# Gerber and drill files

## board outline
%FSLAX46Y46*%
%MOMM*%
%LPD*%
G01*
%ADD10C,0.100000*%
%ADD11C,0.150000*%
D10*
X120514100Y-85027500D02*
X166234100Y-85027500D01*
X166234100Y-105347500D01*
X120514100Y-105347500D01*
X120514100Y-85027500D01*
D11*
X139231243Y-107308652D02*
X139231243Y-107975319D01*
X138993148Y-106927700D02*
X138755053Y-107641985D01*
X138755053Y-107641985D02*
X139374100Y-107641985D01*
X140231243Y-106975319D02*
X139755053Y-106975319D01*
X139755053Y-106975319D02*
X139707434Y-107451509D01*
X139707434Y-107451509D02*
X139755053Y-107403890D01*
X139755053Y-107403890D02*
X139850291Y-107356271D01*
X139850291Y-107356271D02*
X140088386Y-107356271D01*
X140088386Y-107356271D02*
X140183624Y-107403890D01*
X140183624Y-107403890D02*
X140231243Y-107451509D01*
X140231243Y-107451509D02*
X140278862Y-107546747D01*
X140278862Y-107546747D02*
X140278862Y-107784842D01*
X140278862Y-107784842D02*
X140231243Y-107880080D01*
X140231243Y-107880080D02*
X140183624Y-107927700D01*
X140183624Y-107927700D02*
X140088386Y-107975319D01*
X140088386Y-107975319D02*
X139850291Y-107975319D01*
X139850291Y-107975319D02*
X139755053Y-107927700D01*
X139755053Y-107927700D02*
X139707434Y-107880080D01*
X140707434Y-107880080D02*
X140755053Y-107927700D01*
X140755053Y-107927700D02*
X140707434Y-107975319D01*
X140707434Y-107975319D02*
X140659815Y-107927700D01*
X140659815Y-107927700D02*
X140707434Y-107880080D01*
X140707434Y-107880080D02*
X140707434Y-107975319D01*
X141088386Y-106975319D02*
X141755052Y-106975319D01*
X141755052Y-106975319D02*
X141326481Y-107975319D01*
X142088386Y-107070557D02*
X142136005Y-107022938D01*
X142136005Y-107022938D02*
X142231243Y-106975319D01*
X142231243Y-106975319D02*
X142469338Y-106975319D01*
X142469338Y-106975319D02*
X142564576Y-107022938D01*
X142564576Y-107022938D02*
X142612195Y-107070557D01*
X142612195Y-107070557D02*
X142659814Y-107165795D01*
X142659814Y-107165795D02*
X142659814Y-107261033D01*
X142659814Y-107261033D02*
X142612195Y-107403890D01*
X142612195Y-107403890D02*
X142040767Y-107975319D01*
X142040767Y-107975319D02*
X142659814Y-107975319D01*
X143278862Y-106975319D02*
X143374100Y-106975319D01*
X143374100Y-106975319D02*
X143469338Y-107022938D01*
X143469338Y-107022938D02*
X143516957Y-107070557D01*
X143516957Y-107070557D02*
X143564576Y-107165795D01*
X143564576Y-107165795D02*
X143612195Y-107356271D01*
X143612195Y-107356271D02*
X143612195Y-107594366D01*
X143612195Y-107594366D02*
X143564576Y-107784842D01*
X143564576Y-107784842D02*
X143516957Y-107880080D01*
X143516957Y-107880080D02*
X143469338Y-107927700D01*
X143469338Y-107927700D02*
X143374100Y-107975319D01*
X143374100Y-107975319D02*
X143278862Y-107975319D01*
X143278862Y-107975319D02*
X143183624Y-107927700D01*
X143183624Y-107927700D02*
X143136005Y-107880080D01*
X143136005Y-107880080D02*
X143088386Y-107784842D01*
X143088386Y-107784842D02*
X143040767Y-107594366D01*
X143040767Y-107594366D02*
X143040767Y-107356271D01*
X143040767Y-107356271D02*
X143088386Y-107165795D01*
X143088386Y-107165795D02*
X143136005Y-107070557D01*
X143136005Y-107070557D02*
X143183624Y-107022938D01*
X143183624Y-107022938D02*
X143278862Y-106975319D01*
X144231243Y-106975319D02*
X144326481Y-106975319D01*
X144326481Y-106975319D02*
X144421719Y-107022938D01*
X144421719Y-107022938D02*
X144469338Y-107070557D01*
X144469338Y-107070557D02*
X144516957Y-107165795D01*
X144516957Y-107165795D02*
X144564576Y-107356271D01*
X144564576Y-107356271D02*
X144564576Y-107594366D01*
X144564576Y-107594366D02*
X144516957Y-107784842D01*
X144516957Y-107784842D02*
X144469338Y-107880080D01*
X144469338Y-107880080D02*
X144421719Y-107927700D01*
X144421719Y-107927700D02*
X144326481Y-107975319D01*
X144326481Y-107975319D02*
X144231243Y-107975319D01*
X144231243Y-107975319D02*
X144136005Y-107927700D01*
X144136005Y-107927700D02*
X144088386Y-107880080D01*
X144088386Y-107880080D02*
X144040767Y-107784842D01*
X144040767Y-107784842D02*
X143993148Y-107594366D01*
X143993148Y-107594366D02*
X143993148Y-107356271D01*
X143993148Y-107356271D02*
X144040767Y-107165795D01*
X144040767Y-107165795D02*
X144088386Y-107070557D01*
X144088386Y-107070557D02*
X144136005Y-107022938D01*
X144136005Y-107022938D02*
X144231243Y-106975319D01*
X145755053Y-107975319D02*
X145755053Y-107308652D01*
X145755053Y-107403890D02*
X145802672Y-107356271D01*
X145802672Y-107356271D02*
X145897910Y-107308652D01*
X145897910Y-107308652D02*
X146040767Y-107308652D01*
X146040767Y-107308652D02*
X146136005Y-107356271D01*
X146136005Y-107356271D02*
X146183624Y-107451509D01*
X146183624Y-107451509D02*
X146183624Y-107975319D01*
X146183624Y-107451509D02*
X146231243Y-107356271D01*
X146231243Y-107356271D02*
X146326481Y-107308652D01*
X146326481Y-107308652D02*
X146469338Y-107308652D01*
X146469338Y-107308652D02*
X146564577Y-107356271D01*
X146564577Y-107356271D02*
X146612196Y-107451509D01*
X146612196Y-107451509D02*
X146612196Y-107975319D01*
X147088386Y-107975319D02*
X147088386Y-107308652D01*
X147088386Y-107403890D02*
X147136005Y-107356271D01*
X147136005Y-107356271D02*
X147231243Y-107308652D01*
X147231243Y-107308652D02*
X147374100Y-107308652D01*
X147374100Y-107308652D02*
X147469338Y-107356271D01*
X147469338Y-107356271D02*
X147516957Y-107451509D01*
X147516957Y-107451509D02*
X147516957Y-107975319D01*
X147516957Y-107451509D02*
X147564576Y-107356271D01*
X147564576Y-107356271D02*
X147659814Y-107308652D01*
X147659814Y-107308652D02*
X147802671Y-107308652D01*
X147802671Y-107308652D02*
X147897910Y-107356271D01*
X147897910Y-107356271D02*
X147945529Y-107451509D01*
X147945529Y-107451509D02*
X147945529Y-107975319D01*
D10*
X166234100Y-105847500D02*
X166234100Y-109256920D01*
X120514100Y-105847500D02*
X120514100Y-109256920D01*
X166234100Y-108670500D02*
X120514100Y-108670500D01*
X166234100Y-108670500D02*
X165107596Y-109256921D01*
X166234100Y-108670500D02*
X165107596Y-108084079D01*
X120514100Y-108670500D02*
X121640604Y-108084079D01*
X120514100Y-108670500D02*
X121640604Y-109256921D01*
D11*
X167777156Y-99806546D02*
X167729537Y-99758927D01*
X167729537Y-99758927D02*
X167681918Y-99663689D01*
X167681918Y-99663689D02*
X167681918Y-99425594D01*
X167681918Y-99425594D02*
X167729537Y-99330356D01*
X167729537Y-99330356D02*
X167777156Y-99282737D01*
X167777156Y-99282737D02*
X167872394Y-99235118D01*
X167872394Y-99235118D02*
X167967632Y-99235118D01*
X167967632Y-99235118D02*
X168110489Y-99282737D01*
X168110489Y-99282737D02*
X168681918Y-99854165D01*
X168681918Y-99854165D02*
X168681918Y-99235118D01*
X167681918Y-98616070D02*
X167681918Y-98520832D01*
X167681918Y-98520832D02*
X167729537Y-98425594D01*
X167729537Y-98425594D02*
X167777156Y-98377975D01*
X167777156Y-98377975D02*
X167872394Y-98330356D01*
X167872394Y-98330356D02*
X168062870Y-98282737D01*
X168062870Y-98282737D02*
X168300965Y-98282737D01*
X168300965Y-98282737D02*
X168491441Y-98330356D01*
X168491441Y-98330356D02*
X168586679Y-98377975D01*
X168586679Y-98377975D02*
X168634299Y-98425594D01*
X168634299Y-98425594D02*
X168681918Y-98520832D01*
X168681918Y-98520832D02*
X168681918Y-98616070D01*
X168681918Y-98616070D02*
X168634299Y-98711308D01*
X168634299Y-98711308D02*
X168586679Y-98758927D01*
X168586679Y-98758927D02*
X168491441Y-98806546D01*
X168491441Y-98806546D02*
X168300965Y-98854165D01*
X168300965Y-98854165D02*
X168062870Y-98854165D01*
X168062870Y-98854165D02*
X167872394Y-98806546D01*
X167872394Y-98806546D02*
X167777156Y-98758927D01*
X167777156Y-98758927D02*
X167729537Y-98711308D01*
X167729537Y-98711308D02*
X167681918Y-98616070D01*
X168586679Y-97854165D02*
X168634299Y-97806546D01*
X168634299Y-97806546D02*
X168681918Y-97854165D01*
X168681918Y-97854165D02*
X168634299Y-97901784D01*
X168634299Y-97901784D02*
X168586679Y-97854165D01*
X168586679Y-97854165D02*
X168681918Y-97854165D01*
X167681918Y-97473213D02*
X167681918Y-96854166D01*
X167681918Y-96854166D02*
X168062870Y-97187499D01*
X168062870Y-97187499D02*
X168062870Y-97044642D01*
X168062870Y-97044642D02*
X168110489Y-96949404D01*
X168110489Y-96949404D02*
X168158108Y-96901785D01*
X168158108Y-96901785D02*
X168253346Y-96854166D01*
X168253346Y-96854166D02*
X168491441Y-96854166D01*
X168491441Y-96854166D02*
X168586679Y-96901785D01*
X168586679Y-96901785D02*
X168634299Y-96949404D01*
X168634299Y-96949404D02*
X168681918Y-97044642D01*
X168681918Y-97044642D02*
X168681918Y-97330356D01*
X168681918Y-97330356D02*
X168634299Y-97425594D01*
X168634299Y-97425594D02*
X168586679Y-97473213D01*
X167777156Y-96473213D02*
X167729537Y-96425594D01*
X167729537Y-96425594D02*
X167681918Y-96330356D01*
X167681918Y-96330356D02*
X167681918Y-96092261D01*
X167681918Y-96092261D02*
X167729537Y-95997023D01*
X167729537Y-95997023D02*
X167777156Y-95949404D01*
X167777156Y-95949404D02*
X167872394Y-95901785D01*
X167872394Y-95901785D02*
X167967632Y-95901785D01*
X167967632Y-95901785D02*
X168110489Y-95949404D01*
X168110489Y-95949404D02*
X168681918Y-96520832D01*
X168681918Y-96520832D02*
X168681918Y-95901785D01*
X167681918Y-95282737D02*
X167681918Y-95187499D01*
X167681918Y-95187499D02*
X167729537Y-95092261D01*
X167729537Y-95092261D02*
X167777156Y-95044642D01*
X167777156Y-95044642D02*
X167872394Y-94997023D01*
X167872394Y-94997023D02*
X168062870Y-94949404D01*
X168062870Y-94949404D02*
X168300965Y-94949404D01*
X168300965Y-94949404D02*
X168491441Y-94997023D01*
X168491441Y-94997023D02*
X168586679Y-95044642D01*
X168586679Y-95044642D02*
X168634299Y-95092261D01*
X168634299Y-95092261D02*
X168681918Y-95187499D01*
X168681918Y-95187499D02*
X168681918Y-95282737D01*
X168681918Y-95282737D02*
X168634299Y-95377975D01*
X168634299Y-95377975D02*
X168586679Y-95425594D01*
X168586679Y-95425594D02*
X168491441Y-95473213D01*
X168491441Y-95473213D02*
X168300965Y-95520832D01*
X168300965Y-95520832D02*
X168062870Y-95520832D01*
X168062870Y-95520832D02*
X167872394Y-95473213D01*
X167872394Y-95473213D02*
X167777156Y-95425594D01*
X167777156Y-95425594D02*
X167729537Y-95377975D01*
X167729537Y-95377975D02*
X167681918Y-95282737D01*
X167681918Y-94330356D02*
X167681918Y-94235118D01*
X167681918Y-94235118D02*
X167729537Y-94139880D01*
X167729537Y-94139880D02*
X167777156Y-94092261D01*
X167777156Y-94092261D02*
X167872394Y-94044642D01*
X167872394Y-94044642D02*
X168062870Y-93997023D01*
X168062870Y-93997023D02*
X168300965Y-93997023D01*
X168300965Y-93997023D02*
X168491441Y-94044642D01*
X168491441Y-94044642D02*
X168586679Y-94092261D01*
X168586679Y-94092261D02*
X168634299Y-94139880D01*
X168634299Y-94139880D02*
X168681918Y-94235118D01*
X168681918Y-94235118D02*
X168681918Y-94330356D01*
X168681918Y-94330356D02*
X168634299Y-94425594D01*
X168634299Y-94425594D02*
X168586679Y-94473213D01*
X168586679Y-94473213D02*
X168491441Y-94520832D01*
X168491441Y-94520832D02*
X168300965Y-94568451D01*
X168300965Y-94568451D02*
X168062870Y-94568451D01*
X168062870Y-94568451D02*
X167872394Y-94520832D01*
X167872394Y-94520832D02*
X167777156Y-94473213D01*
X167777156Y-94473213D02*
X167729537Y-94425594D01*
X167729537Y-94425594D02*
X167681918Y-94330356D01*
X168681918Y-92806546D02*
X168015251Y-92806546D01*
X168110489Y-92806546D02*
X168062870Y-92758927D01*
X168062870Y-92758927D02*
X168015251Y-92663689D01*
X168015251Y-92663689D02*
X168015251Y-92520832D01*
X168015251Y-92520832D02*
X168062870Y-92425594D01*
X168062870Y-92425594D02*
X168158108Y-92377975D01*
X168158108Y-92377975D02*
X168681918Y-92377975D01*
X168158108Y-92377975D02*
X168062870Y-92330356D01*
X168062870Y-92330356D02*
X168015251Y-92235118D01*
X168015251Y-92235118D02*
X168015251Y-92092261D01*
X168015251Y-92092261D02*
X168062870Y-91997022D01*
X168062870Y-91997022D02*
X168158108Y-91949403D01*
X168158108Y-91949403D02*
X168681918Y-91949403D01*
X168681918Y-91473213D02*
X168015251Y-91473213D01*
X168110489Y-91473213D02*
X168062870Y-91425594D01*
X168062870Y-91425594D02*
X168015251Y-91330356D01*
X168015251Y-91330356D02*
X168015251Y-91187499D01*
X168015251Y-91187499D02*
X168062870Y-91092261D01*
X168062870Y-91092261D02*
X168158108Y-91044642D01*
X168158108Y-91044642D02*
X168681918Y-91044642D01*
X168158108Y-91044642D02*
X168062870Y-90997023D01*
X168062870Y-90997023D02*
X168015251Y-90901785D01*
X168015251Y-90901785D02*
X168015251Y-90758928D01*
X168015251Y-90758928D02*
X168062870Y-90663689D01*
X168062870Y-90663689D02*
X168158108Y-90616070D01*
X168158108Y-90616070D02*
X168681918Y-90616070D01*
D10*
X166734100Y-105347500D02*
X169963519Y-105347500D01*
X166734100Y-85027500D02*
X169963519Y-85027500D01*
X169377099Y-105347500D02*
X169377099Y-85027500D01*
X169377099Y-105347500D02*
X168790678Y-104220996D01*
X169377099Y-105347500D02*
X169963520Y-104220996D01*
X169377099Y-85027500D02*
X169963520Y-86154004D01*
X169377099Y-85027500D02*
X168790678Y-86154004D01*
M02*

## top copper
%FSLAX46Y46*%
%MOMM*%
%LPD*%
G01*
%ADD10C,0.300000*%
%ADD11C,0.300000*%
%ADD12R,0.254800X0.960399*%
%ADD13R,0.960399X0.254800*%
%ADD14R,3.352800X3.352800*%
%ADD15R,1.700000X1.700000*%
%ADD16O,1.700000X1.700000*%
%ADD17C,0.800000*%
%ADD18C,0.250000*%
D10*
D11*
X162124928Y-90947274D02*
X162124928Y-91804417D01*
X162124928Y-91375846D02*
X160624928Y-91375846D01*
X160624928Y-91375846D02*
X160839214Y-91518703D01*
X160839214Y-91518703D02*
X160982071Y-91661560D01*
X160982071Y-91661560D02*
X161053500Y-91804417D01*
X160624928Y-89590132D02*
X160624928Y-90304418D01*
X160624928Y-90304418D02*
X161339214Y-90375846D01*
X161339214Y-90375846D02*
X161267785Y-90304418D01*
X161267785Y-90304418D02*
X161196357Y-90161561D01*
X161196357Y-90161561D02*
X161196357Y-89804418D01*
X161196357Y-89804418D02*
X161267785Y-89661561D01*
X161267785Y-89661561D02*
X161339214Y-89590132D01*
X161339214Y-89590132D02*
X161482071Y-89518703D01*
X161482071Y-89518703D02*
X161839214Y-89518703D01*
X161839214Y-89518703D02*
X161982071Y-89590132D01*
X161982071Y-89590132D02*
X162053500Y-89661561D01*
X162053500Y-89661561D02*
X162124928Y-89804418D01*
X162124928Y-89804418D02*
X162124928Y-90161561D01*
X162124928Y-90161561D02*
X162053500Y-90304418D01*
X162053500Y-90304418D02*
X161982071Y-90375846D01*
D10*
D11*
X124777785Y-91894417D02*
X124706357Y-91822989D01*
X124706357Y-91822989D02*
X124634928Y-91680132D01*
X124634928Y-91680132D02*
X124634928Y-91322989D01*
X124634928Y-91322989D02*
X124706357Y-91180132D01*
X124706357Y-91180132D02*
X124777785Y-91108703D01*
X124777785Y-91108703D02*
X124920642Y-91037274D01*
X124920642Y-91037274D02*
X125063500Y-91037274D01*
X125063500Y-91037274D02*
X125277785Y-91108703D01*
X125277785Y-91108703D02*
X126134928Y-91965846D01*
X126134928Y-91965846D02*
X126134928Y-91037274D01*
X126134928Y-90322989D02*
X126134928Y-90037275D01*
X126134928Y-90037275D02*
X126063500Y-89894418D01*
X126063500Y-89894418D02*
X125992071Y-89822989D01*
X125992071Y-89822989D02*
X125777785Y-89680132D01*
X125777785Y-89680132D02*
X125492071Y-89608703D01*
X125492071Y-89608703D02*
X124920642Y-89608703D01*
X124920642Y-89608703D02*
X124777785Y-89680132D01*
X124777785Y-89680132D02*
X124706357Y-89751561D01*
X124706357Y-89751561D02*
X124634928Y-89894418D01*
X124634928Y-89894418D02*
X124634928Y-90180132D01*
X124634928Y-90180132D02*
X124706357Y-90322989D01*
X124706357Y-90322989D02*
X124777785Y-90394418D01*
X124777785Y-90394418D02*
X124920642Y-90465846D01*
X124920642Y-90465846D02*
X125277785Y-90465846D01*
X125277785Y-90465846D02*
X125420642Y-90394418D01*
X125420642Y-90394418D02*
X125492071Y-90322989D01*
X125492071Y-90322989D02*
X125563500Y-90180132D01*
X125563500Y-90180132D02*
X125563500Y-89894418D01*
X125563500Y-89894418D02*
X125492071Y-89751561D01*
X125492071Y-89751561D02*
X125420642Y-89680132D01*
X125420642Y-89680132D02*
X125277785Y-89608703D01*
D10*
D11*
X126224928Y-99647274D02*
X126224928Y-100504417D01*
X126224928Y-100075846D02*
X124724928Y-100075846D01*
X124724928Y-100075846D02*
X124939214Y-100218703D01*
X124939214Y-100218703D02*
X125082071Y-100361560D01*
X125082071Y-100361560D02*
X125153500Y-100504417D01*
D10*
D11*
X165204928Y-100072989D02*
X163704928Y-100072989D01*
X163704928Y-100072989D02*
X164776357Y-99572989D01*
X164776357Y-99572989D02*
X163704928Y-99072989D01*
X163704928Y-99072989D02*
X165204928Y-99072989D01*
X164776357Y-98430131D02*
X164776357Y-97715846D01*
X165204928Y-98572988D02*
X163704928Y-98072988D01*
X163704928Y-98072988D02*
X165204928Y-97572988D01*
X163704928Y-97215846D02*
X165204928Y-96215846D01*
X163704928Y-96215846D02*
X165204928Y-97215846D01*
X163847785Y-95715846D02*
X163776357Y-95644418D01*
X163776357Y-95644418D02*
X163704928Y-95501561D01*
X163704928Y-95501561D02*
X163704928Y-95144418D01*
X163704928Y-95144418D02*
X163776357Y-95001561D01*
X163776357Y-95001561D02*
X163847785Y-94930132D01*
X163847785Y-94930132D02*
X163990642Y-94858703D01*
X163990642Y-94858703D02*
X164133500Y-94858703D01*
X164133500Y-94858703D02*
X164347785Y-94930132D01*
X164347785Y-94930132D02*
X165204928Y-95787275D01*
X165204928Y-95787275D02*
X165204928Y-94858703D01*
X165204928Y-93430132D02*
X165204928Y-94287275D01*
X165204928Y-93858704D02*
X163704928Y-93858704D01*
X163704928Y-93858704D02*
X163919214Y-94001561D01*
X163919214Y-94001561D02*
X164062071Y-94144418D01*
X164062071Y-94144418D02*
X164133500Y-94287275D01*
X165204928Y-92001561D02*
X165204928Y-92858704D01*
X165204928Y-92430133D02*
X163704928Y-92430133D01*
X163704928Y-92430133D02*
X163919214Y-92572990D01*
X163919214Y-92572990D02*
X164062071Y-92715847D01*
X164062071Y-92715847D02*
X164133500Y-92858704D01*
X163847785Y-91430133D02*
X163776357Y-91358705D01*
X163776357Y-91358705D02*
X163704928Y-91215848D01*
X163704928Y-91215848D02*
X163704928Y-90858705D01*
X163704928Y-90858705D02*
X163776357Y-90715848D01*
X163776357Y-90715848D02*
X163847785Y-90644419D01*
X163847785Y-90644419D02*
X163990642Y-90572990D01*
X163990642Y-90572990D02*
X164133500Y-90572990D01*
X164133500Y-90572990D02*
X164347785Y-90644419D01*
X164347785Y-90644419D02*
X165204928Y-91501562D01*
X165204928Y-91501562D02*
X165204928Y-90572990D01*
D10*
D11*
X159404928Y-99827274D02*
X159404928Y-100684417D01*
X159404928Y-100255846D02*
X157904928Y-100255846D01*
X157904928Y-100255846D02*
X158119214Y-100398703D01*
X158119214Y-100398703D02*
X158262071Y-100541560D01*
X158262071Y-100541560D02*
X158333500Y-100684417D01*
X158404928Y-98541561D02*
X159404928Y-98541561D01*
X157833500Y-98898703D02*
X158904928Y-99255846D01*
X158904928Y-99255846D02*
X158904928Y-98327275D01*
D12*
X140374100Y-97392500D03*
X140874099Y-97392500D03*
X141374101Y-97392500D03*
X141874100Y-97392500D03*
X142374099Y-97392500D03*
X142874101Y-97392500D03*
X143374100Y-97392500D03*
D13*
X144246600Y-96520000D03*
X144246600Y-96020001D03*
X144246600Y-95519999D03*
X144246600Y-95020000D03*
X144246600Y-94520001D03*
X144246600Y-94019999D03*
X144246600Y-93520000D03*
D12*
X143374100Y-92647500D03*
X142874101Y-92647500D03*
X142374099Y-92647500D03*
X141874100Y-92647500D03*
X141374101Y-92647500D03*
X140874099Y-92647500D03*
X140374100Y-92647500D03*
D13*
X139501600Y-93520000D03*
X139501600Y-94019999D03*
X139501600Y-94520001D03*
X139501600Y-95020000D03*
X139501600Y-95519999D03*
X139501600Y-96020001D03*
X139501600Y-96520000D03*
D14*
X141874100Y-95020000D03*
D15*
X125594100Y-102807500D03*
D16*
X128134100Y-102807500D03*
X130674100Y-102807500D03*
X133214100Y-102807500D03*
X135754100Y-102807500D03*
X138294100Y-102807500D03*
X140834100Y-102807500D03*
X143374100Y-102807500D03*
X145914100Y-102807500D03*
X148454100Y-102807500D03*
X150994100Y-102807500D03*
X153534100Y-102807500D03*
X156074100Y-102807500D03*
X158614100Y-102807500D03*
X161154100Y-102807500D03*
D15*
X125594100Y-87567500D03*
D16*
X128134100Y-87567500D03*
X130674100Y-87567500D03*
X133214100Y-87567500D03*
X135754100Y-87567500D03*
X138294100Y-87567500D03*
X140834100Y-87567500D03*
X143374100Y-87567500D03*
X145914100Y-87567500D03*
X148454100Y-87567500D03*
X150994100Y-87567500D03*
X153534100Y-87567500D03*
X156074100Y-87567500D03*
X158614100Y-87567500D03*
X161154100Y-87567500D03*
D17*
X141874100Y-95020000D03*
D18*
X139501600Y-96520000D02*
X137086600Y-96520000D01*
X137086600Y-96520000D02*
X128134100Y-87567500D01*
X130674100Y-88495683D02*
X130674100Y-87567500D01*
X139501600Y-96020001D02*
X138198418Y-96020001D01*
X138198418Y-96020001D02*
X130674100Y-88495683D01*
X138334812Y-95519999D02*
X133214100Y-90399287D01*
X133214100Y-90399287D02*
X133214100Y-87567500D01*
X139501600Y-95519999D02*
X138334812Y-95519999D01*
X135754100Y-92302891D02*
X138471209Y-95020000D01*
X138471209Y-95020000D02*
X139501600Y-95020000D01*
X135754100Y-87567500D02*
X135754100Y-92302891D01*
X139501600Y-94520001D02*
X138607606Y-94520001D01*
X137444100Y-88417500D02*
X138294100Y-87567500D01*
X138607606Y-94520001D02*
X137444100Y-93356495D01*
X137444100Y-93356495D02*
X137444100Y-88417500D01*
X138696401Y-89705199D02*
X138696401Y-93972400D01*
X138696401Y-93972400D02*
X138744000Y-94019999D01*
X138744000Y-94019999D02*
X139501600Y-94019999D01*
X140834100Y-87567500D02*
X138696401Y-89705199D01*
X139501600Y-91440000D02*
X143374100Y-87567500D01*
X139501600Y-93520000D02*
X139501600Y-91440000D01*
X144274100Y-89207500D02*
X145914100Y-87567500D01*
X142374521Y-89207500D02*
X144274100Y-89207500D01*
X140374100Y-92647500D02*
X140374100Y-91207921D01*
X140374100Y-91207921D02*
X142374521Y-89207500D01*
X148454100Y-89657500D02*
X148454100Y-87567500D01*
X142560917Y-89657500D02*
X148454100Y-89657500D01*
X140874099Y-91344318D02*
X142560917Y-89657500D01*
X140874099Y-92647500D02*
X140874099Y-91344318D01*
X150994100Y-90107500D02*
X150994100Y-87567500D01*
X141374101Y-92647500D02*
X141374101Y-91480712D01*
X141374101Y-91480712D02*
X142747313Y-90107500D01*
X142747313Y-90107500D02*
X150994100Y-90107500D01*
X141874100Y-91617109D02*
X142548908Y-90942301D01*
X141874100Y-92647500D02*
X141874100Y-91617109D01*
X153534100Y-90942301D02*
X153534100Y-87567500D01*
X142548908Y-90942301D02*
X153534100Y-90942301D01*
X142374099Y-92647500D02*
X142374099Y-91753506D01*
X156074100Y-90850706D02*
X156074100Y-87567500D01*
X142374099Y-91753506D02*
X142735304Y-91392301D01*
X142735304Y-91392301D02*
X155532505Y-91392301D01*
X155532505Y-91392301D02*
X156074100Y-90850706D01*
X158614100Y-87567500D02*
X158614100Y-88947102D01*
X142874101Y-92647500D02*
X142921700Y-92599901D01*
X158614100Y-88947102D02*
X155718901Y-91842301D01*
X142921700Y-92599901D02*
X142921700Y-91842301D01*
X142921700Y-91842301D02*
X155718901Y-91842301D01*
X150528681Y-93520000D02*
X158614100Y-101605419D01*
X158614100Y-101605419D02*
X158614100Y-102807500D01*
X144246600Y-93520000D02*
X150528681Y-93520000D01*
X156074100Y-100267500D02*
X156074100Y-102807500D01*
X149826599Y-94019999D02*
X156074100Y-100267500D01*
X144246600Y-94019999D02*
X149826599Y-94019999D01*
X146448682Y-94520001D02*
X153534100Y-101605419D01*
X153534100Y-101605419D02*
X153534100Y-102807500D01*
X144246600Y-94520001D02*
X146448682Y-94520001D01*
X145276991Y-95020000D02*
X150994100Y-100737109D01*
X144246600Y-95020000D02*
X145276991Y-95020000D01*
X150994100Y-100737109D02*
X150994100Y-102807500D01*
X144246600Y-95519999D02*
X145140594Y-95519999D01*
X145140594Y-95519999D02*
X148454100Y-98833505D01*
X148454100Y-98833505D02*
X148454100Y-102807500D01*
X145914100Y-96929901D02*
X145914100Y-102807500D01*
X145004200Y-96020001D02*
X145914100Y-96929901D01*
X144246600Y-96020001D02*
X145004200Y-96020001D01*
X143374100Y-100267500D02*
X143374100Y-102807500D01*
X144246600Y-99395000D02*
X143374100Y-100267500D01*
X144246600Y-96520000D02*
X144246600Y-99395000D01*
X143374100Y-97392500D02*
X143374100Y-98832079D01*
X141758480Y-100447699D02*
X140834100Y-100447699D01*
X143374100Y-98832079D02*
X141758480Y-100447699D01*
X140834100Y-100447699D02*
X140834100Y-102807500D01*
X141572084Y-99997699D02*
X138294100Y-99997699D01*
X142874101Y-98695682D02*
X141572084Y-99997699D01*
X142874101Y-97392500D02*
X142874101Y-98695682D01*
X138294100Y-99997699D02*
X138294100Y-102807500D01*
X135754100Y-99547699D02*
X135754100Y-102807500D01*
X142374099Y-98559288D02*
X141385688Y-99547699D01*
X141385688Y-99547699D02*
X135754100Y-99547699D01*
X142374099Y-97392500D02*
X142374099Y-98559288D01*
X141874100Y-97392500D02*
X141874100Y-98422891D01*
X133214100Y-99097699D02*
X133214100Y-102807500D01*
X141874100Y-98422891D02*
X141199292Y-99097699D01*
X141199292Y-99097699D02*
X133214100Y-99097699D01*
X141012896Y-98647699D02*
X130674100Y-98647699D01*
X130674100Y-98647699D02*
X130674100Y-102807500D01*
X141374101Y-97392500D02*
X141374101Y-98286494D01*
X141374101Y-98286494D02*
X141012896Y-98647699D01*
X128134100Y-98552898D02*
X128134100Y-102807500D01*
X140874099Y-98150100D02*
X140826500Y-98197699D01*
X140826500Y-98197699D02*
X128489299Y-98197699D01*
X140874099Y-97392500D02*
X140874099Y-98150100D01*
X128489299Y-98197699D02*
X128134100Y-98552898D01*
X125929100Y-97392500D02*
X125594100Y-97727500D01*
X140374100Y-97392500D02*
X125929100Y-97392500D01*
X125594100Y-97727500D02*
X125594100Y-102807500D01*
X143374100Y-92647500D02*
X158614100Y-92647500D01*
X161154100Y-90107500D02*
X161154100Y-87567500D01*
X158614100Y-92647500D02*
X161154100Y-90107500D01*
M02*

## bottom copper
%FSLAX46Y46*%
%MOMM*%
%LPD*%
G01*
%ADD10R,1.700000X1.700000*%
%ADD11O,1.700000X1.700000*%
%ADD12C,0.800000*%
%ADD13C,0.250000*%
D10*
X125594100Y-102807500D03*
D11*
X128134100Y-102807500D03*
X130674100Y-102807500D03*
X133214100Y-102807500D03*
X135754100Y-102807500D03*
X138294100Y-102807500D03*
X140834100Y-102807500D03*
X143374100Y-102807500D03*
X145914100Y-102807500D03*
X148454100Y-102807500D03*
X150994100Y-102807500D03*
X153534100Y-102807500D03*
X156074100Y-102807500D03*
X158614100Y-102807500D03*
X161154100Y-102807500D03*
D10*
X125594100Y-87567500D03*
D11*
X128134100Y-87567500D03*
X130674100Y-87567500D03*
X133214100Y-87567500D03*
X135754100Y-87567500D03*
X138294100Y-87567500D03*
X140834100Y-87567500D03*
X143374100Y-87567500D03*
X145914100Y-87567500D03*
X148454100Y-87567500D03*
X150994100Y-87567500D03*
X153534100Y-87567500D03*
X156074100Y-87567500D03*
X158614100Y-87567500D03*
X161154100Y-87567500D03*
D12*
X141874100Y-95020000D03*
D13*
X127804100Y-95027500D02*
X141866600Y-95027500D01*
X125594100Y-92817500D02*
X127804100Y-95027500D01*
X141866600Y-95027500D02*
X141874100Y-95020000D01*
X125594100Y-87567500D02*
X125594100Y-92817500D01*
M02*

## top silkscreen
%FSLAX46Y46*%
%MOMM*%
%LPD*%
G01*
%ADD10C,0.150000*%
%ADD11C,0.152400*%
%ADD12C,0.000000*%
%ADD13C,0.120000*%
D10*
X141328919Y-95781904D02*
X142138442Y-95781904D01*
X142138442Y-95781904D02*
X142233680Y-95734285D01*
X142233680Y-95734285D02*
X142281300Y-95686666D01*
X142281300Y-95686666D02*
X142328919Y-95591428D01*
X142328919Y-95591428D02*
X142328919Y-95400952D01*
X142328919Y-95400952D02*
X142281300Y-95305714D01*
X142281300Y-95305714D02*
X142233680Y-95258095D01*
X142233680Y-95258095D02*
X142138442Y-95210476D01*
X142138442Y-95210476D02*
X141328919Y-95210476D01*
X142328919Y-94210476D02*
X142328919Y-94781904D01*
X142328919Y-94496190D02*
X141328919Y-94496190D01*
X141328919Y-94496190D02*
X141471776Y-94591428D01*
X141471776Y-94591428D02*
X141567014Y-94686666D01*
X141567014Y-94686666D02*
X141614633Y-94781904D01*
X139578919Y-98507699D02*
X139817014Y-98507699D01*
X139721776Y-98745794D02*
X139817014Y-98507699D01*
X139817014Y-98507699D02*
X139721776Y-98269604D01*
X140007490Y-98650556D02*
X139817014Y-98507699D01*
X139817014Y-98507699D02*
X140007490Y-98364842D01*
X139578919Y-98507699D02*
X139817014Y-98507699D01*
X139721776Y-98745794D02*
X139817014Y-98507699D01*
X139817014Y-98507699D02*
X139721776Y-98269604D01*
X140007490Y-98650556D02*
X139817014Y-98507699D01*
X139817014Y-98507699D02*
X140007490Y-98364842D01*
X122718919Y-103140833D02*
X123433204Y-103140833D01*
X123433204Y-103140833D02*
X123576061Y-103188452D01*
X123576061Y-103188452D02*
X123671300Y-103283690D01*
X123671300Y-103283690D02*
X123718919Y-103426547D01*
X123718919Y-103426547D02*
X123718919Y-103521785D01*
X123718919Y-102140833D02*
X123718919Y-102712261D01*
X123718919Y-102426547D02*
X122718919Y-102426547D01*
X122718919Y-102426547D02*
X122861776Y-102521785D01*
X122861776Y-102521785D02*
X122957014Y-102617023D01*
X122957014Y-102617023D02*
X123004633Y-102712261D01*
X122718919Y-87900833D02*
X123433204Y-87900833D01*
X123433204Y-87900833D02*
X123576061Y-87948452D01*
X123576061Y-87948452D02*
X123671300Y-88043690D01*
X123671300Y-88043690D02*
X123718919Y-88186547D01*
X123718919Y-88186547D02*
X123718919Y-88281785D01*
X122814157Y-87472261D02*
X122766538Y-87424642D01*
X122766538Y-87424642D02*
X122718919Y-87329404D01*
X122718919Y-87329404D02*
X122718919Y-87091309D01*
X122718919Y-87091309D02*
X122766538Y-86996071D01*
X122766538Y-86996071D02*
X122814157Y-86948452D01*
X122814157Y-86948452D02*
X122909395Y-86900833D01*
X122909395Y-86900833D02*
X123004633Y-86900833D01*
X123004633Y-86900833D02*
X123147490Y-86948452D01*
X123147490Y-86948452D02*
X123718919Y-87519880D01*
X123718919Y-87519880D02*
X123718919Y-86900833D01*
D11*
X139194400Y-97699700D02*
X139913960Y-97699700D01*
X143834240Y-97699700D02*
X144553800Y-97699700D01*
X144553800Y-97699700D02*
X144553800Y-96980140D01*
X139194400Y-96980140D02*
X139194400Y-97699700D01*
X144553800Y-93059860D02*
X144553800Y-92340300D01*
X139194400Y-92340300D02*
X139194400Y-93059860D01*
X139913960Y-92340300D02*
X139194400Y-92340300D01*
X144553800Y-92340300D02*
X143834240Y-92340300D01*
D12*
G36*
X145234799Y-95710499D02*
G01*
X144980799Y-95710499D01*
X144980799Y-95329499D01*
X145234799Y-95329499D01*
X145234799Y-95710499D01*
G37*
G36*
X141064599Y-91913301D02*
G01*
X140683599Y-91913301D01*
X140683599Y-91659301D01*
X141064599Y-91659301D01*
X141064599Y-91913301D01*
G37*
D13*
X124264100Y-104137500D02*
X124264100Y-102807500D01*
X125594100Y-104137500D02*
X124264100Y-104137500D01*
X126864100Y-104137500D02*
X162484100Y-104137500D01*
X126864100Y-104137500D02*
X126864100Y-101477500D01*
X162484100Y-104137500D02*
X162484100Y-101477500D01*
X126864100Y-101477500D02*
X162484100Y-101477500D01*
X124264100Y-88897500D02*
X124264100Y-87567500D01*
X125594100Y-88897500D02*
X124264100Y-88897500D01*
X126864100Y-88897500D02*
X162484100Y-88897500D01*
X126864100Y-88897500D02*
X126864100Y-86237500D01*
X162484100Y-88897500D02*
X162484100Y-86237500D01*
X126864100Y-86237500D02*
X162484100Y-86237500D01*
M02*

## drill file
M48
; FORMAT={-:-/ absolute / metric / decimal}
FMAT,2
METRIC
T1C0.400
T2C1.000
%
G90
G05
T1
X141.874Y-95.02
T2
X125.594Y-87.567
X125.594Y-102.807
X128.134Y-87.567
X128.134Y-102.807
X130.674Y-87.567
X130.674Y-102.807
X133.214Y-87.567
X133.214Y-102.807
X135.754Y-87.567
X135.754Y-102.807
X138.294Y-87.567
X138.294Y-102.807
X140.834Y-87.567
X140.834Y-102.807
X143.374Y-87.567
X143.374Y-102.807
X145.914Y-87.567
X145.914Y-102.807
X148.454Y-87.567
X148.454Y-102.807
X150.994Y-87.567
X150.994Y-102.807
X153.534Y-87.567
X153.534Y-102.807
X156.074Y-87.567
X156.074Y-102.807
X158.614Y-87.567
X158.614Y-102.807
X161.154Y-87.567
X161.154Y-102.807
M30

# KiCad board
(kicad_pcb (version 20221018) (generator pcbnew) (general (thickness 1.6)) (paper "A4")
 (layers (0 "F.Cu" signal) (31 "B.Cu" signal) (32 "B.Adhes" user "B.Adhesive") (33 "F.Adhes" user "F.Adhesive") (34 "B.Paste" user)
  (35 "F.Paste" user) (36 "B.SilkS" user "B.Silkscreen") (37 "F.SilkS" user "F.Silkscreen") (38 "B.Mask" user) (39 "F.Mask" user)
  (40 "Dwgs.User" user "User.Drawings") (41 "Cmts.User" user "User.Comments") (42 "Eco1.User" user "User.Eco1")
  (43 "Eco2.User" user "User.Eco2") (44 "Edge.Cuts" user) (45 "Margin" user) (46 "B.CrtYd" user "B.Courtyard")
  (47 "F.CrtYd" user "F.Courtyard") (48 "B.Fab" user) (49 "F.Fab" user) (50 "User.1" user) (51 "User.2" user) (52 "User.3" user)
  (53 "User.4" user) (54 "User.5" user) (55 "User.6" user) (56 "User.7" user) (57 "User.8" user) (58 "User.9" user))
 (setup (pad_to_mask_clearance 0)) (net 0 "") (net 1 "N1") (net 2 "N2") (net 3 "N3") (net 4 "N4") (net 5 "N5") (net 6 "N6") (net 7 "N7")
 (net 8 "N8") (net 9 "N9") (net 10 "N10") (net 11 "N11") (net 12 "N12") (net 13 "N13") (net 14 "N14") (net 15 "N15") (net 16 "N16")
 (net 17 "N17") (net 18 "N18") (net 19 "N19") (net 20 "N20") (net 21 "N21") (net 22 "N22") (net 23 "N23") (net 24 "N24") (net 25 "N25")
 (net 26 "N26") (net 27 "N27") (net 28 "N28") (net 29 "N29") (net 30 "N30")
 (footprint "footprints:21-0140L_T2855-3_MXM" (layer "F.Cu") (at 141.8741 95.02 90)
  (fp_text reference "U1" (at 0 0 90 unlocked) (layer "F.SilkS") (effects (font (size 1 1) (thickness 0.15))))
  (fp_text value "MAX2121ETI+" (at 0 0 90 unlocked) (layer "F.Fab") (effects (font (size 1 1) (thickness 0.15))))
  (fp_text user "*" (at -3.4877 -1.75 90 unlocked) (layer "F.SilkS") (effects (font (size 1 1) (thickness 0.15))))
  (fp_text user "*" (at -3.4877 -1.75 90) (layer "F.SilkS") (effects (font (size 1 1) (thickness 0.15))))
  (fp_line (start -2.6797 -2.6797) (end -2.6797 -1.96014) (stroke (width 0.1524) (type solid)) (layer "F.SilkS"))
  (fp_line (start -2.6797 1.96014) (end -2.6797 2.6797) (stroke (width 0.1524) (type solid)) (layer "F.SilkS"))
  (fp_line (start -2.6797 2.6797) (end -1.96014 2.6797) (stroke (width 0.1524) (type solid)) (layer "F.SilkS"))
  (fp_line (start -1.96014 -2.6797) (end -2.6797 -2.6797) (stroke (width 0.1524) (type solid)) (layer "F.SilkS"))
  (fp_line (start 1.96014 2.6797) (end 2.6797 2.6797) (stroke (width 0.1524) (type solid)) (layer "F.SilkS"))
  (fp_line (start 2.6797 -2.6797) (end 1.96014 -2.6797) (stroke (width 0.1524) (type solid)) (layer "F.SilkS"))
  (fp_line (start 2.6797 -1.96014) (end 2.6797 -2.6797) (stroke (width 0.1524) (type solid)) (layer "F.SilkS"))
  (fp_line (start 2.6797 2.6797) (end 2.6797 1.96014) (stroke (width 0.1524) (type solid)) (layer "F.SilkS"))
  (fp_poly
   (pts (xy -0.690499 3.106699) (xy -0.690499 3.360699) (xy -0.309499 3.360699) (xy -0.309499 3.106699)) (stroke (width 0) (type solid))
   (fill solid) (layer "F.SilkS"))
  (fp_poly
   (pts (xy 3.360699 -1.190501) (xy 3.360699 -0.809501) (xy 3.106699 -0.809501) (xy 3.106699 -1.190501)) (stroke (width 0) (type solid))
   (fill solid) (layer "F.SilkS"))
  (pad "1" smd rect (at -2.3725 -1.5 180) (size 0.2548 0.960399) (layers "F.Cu" "F.Paste" "F.Mask") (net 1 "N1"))
  (pad "2" smd rect (at -2.3725 -1.000001 180) (size 0.2548 0.960399) (layers "F.Cu" "F.Paste" "F.Mask") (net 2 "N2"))
  (pad "3" smd rect (at -2.3725 -0.499999 180) (size 0.2548 0.960399) (layers "F.Cu" "F.Paste" "F.Mask") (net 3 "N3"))
  (pad "4" smd rect (at -2.3725 0 180) (size 0.2548 0.960399) (layers "F.Cu" "F.Paste" "F.Mask") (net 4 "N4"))
  (pad "5" smd rect (at -2.3725 0.499999 180) (size 0.2548 0.960399) (layers "F.Cu" "F.Paste" "F.Mask") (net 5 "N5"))
  (pad "6" smd rect (at -2.3725 1.000001 180) (size 0.2548 0.960399) (layers "F.Cu" "F.Paste" "F.Mask") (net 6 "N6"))
  (pad "7" smd rect (at -2.3725 1.5 180) (size 0.2548 0.960399) (layers "F.Cu" "F.Paste" "F.Mask") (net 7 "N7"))
  (pad "8" smd rect (at -1.5 2.3725 90) (size 0.2548 0.960399) (layers "F.Cu" "F.Paste" "F.Mask") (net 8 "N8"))
  (pad "9" smd rect (at -1.000001 2.3725 90) (size 0.2548 0.960399) (layers "F.Cu" "F.Paste" "F.Mask") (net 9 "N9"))
  (pad "10" smd rect (at -0.499999 2.3725 90) (size 0.2548 0.960399) (layers "F.Cu" "F.Paste" "F.Mask") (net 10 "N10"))
  (pad "11" smd rect (at 0 2.3725 90) (size 0.2548 0.960399) (layers "F.Cu" "F.Paste" "F.Mask") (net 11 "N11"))
  (pad "12" smd rect (at 0.499999 2.3725 90) (size 0.2548 0.960399) (layers "F.Cu" "F.Paste" "F.Mask") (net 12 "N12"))
  (pad "13" smd rect (at 1.000001 2.3725 90) (size 0.2548 0.960399) (layers "F.Cu" "F.Paste" "F.Mask") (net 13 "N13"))
  (pad "14" smd rect (at 1.5 2.3725 90) (size 0.2548 0.960399) (layers "F.Cu" "F.Paste" "F.Mask") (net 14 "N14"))
  (pad "15" smd rect (at 2.3725 1.5 180) (size 0.2548 0.960399) (layers "F.Cu" "F.Paste" "F.Mask") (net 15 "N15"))
  (pad "16" smd rect (at 2.3725 1.000001 180) (size 0.2548 0.960399) (layers "F.Cu" "F.Paste" "F.Mask") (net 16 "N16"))
  (pad "17" smd rect (at 2.3725 0.499999 180) (size 0.2548 0.960399) (layers "F.Cu" "F.Paste" "F.Mask") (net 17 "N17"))
  (pad "18" smd rect (at 2.3725 0 180) (size 0.2548 0.960399) (layers "F.Cu" "F.Paste" "F.Mask") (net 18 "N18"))
  (pad "19" smd rect (at 2.3725 -0.499999 180) (size 0.2548 0.960399) (layers "F.Cu" "F.Paste" "F.Mask") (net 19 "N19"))
  (pad "20" smd rect (at 2.3725 -1.000001 180) (size 0.2548 0.960399) (layers "F.Cu" "F.Paste" "F.Mask") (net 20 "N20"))
  (pad "21" smd rect (at 2.3725 -1.5 180) (size 0.2548 0.960399) (layers "F.Cu" "F.Paste" "F.Mask") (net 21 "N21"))
  (pad "22" smd rect (at 1.5 -2.3725 90) (size 0.2548 0.960399) (layers "F.Cu" "F.Paste" "F.Mask") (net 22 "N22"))
  (pad "23" smd rect (at 1.000001 -2.3725 90) (size 0.2548 0.960399) (layers "F.Cu" "F.Paste" "F.Mask") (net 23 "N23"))
  (pad "24" smd rect (at 0.499999 -2.3725 90) (size 0.2548 0.960399) (layers "F.Cu" "F.Paste" "F.Mask") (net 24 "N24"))
  (pad "25" smd rect (at 0 -2.3725 90) (size 0.2548 0.960399) (layers "F.Cu" "F.Paste" "F.Mask") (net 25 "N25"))
  (pad "26" smd rect (at -0.499999 -2.3725 90) (size 0.2548 0.960399) (layers "F.Cu" "F.Paste" "F.Mask") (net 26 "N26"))
  (pad "27" smd rect (at -1.000001 -2.3725 90) (size 0.2548 0.960399) (layers "F.Cu" "F.Paste" "F.Mask") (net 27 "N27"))
  (pad "28" smd rect (at -1.5 -2.3725 90) (size 0.2548 0.960399) (layers "F.Cu" "F.Paste" "F.Mask") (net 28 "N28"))
  (pad "29" smd rect (at 0 0 90) (size 3.3528 3.3528) (layers "F.Cu" "F.Mask") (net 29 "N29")))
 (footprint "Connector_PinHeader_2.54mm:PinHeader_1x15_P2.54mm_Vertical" (layer "F.Cu") (at 125.5941 102.8075 90)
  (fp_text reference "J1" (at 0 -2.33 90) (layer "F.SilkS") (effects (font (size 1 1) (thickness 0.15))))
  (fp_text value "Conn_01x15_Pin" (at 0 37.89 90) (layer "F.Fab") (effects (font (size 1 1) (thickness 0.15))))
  (fp_line (start -1.33 -1.33) (end 0 -1.33) (stroke (width 0.12) (type solid)) (layer "F.SilkS"))
  (fp_line (start -1.33 0) (end -1.33 -1.33) (stroke (width 0.12) (type solid)) (layer "F.SilkS"))
  (fp_line (start -1.33 1.27) (end -1.33 36.89) (stroke (width 0.12) (type solid)) (layer "F.SilkS"))
  (fp_line (start -1.33 1.27) (end 1.33 1.27) (stroke (width 0.12) (type solid)) (layer "F.SilkS"))
  (fp_line (start -1.33 36.89) (end 1.33 36.89) (stroke (width 0.12) (type solid)) (layer "F.SilkS"))
  (fp_line (start 1.33 1.27) (end 1.33 36.89) (stroke (width 0.12) (type solid)) (layer "F.SilkS"))
  (pad "1" thru_hole rect (at 0 0 90) (size 1.7 1.7) (drill 1) (layers "*.Cu" "*.Mask") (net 1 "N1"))
  (pad "2" thru_hole oval (at 0 2.54 90) (size 1.7 1.7) (drill 1) (layers "*.Cu" "*.Mask") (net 2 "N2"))
  (pad "3" thru_hole oval (at 0 5.08 90) (size 1.7 1.7) (drill 1) (layers "*.Cu" "*.Mask") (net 3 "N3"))
  (pad "4" thru_hole oval (at 0 7.62 90) (size 1.7 1.7) (drill 1) (layers "*.Cu" "*.Mask") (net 4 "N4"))
  (pad "5" thru_hole oval (at 0 10.16 90) (size 1.7 1.7) (drill 1) (layers "*.Cu" "*.Mask") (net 5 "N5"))
  (pad "6" thru_hole oval (at 0 12.7 90) (size 1.7 1.7) (drill 1) (layers "*.Cu" "*.Mask") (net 6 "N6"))
  (pad "7" thru_hole oval (at 0 15.24 90) (size 1.7 1.7) (drill 1) (layers "*.Cu" "*.Mask") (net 7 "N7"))
  (pad "8" thru_hole oval (at 0 17.78 90) (size 1.7 1.7) (drill 1) (layers "*.Cu" "*.Mask") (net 8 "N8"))
  (pad "9" thru_hole oval (at 0 20.32 90) (size 1.7 1.7) (drill 1) (layers "*.Cu" "*.Mask") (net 9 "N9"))
  (pad "10" thru_hole oval (at 0 22.86 90) (size 1.7 1.7) (drill 1) (layers "*.Cu" "*.Mask") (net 10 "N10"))
  (pad "11" thru_hole oval (at 0 25.4 90) (size 1.7 1.7) (drill 1) (layers "*.Cu" "*.Mask") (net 11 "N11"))
  (pad "12" thru_hole oval (at 0 27.94 90) (size 1.7 1.7) (drill 1) (layers "*.Cu" "*.Mask") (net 12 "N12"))
  (pad "13" thru_hole oval (at 0 30.48 90) (size 1.7 1.7) (drill 1) (layers "*.Cu" "*.Mask") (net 13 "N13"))
  (pad "14" thru_hole oval (at 0 33.02 90) (size 1.7 1.7) (drill 1) (layers "*.Cu" "*.Mask") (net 14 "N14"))
  (pad "15" thru_hole oval (at 0 35.56 90) (size 1.7 1.7) (drill 1) (layers "*.Cu" "*.Mask") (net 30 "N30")))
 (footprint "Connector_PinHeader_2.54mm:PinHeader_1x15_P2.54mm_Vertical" (layer "F.Cu") (at 125.5941 87.5675 90)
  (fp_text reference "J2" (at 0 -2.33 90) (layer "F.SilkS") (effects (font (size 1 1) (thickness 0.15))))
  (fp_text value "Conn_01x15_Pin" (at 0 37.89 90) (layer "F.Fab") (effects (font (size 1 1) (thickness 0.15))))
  (fp_line (start -1.33 -1.33) (end 0 -1.33) (stroke (width 0.12) (type solid)) (layer "F.SilkS"))
  (fp_line (start -1.33 0) (end -1.33 -1.33) (stroke (width 0.12) (type solid)) (layer "F.SilkS"))
  (fp_line (start -1.33 1.27) (end -1.33 36.89) (stroke (width 0.12) (type solid)) (layer "F.SilkS"))
  (fp_line (start -1.33 1.27) (end 1.33 1.27) (stroke (width 0.12) (type solid)) (layer "F.SilkS"))
  (fp_line (start -1.33 36.89) (end 1.33 36.89) (stroke (width 0.12) (type solid)) (layer "F.SilkS"))
  (fp_line (start 1.33 1.27) (end 1.33 36.89) (stroke (width 0.12) (type solid)) (layer "F.SilkS"))
  (pad "1" thru_hole rect (at 0 0 90) (size 1.7 1.7) (drill 1) (layers "*.Cu" "*.Mask") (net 29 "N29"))
  (pad "2" thru_hole oval (at 0 2.54 90) (size 1.7 1.7) (drill 1) (layers "*.Cu" "*.Mask") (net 28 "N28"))
  (pad "3" thru_hole oval (at 0 5.08 90) (size 1.7 1.7) (drill 1) (layers "*.Cu" "*.Mask") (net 27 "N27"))
  (pad "4" thru_hole oval (at 0 7.62 90) (size 1.7 1.7) (drill 1) (layers "*.Cu" "*.Mask") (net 26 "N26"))
  (pad "5" thru_hole oval (at 0 10.16 90) (size 1.7 1.7) (drill 1) (layers "*.Cu" "*.Mask") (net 25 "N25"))
  (pad "6" thru_hole oval (at 0 12.7 90) (size 1.7 1.7) (drill 1) (layers "*.Cu" "*.Mask") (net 24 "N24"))
  (pad "7" thru_hole oval (at 0 15.24 90) (size 1.7 1.7) (drill 1) (layers "*.Cu" "*.Mask") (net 23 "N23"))
  (pad "8" thru_hole oval (at 0 17.78 90) (size 1.7 1.7) (drill 1) (layers "*.Cu" "*.Mask") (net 22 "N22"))
  (pad "9" thru_hole oval (at 0 20.32 90) (size 1.7 1.7) (drill 1) (layers "*.Cu" "*.Mask") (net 21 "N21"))
  (pad "10" thru_hole oval (at 0 22.86 90) (size 1.7 1.7) (drill 1) (layers "*.Cu" "*.Mask") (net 20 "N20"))
  (pad "11" thru_hole oval (at 0 25.4 90) (size 1.7 1.7) (drill 1) (layers "*.Cu" "*.Mask") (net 19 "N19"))
  (pad "12" thru_hole oval (at 0 27.94 90) (size 1.7 1.7) (drill 1) (layers "*.Cu" "*.Mask") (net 18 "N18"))
  (pad "13" thru_hole oval (at 0 30.48 90) (size 1.7 1.7) (drill 1) (layers "*.Cu" "*.Mask") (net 17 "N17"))
  (pad "14" thru_hole oval (at 0 33.02 90) (size 1.7 1.7) (drill 1) (layers "*.Cu" "*.Mask") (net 16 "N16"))
  (pad "15" thru_hole oval (at 0 35.56 90) (size 1.7 1.7) (drill 1) (layers "*.Cu" "*.Mask") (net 15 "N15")))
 (gr_rect (start 120.5141 105.3475) (end 166.2341 85.0275) (stroke (width 0.1) (type default)) (fill none) (layer "Edge.Cuts"))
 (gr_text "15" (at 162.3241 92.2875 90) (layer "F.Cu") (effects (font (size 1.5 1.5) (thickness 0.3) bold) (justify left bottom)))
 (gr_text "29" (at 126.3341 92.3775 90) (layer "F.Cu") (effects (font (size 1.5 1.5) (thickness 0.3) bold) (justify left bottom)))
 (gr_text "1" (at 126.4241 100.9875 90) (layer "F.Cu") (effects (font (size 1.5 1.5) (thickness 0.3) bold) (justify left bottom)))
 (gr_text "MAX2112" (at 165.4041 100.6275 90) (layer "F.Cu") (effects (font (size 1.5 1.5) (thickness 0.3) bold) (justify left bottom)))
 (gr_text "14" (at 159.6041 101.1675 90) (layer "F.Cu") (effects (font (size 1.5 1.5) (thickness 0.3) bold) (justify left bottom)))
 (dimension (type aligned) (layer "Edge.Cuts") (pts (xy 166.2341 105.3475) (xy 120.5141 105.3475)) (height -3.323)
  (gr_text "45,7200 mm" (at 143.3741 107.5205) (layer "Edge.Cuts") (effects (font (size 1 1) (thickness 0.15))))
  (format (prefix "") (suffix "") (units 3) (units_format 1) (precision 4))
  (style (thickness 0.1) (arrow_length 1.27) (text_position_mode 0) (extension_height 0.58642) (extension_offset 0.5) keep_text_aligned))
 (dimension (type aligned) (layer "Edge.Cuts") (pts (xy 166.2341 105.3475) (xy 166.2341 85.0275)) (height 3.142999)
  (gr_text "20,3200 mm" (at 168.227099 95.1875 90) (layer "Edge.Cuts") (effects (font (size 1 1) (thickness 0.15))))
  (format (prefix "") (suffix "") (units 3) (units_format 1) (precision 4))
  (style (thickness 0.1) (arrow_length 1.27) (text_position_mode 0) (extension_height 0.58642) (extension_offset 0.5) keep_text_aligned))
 (via (at 141.8741 95.02) (size 0.8) (drill 0.4) (layers "F.Cu" "B.Cu") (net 29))
 (segment (start 127.8041 95.0275) (end 141.8666 95.0275) (width 0.25) (layer "B.Cu") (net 29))
 (segment (start 125.5941 92.8175) (end 127.8041 95.0275) (width 0.25) (layer "B.Cu") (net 29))
 (segment (start 141.8666 95.0275) (end 141.8741 95.02) (width 0.25) (layer "B.Cu") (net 29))
 (segment (start 125.5941 87.5675) (end 125.5941 92.8175) (width 0.25) (layer "B.Cu") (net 29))
 (segment (start 139.5016 96.52) (end 137.0866 96.52) (width 0.25) (layer "F.Cu") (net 28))
 (segment (start 137.0866 96.52) (end 128.1341 87.5675) (width 0.25) (layer "F.Cu") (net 28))
 (segment (start 130.6741 88.495683) (end 130.6741 87.5675) (width 0.25) (layer "F.Cu") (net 27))
 (segment (start 139.5016 96.020001) (end 138.198418 96.020001) (width 0.25) (layer "F.Cu") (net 27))
 (segment (start 138.198418 96.020001) (end 130.6741 88.495683) (width 0.25) (layer "F.Cu") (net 27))
 (segment (start 138.334812 95.519999) (end 133.2141 90.399287) (width 0.25) (layer "F.Cu") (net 26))
 (segment (start 133.2141 90.399287) (end 133.2141 87.5675) (width 0.25) (layer "F.Cu") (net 26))
 (segment (start 139.5016 95.519999) (end 138.334812 95.519999) (width 0.25) (layer "F.Cu") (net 26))
 (segment (start 135.7541 92.302891) (end 138.471209 95.02) (width 0.25) (layer "F.Cu") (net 25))
 (segment (start 138.471209 95.02) (end 139.5016 95.02) (width 0.25) (layer "F.Cu") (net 25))
 (segment (start 135.7541 87.5675) (end 135.7541 92.302891) (width 0.25) (layer "F.Cu") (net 25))
 (segment (start 139.5016 94.520001) (end 138.607606 94.520001) (width 0.25) (layer "F.Cu") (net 24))
 (segment (start 137.4441 88.4175) (end 138.2941 87.5675) (width 0.25) (layer "F.Cu") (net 24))
 (segment (start 138.607606 94.520001) (end 137.4441 93.356495) (width 0.25) (layer "F.Cu") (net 24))
 (segment (start 137.4441 93.356495) (end 137.4441 88.4175) (width 0.25) (layer "F.Cu") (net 24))
 (segment (start 138.696401 89.705199) (end 138.696401 93.9724) (width 0.25) (layer "F.Cu") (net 23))
 (segment (start 138.696401 93.9724) (end 138.744 94.019999) (width 0.25) (layer "F.Cu") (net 23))
 (segment (start 138.744 94.019999) (end 139.5016 94.019999) (width 0.25) (layer "F.Cu") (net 23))
 (segment (start 140.8341 87.5675) (end 138.696401 89.705199) (width 0.25) (layer "F.Cu") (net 23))
 (segment (start 139.5016 91.44) (end 143.3741 87.5675) (width 0.25) (layer "F.Cu") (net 22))
 (segment (start 139.5016 93.52) (end 139.5016 91.44) (width 0.25) (layer "F.Cu") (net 22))
 (segment (start 144.2741 89.2075) (end 145.9141 87.5675) (width 0.25) (layer "F.Cu") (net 21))
 (segment (start 142.374521 89.2075) (end 144.2741 89.2075) (width 0.25) (layer "F.Cu") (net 21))
 (segment (start 140.3741 92.6475) (end 140.3741 91.207921) (width 0.25) (layer "F.Cu") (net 21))
 (segment (start 140.3741 91.207921) (end 142.374521 89.2075) (width 0.25) (layer "F.Cu") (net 21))
 (segment (start 148.4541 89.6575) (end 148.4541 87.5675) (width 0.25) (layer "F.Cu") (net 20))
 (segment (start 142.560917 89.6575) (end 148.4541 89.6575) (width 0.25) (layer "F.Cu") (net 20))
 (segment (start 140.874099 91.344318) (end 142.560917 89.6575) (width 0.25) (layer "F.Cu") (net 20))
 (segment (start 140.874099 92.6475) (end 140.874099 91.344318) (width 0.25) (layer "F.Cu") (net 20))
 (segment (start 150.9941 90.1075) (end 150.9941 87.5675) (width 0.25) (layer "F.Cu") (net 19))
 (segment (start 141.374101 92.6475) (end 141.374101 91.480712) (width 0.25) (layer "F.Cu") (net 19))
 (segment (start 141.374101 91.480712) (end 142.747313 90.1075) (width 0.25) (layer "F.Cu") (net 19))
 (segment (start 142.747313 90.1075) (end 150.9941 90.1075) (width 0.25) (layer "F.Cu") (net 19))
 (segment (start 141.8741 91.617109) (end 142.548908 90.942301) (width 0.25) (layer "F.Cu") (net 18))
 (segment (start 141.8741 92.6475) (end 141.8741 91.617109) (width 0.25) (layer "F.Cu") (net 18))
 (segment (start 153.5341 90.942301) (end 153.5341 87.5675) (width 0.25) (layer "F.Cu") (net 18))
 (segment (start 142.548908 90.942301) (end 153.5341 90.942301) (width 0.25) (layer "F.Cu") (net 18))
 (segment (start 142.374099 92.6475) (end 142.374099 91.753506) (width 0.25) (layer "F.Cu") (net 17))
 (segment (start 156.0741 90.850706) (end 156.0741 87.5675) (width 0.25) (layer "F.Cu") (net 17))
 (segment (start 142.374099 91.753506) (end 142.735304 91.392301) (width 0.25) (layer "F.Cu") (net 17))
 (segment (start 142.735304 91.392301) (end 155.532505 91.392301) (width 0.25) (layer "F.Cu") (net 17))
 (segment (start 155.532505 91.392301) (end 156.0741 90.850706) (width 0.25) (layer "F.Cu") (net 17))
 (segment (start 158.6141 87.5675) (end 158.6141 88.947102) (width 0.25) (layer "F.Cu") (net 16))
 (segment (start 142.874101 92.6475) (end 142.9217 92.599901) (width 0.25) (layer "F.Cu") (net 16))
 (segment (start 158.6141 88.947102) (end 155.718901 91.842301) (width 0.25) (layer "F.Cu") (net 16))
 (segment (start 142.9217 92.599901) (end 142.9217 91.842301) (width 0.25) (layer "F.Cu") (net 16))
 (segment (start 142.9217 91.842301) (end 155.718901 91.842301) (width 0.25) (layer "F.Cu") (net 16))
 (segment (start 150.528681 93.52) (end 158.6141 101.605419) (width 0.25) (layer "F.Cu") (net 14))
 (segment (start 158.6141 101.605419) (end 158.6141 102.8075) (width 0.25) (layer "F.Cu") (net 14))
 (segment (start 144.2466 93.52) (end 150.528681 93.52) (width 0.25) (layer "F.Cu") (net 14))
 (segment (start 156.0741 100.2675) (end 156.0741 102.8075) (width 0.25) (layer "F.Cu") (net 13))
 (segment (start 149.826599 94.019999) (end 156.0741 100.2675) (width 0.25) (layer "F.Cu") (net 13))
 (segment (start 144.2466 94.019999) (end 149.826599 94.019999) (width 0.25) (layer "F.Cu") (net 13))
 (segment (start 146.448682 94.520001) (end 153.5341 101.605419) (width 0.25) (layer "F.Cu") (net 12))
 (segment (start 153.5341 101.605419) (end 153.5341 102.8075) (width 0.25) (layer "F.Cu") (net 12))
 (segment (start 144.2466 94.520001) (end 146.448682 94.520001) (width 0.25) (layer "F.Cu") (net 12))
 (segment (start 145.276991 95.02) (end 150.9941 100.737109) (width 0.25) (layer "F.Cu") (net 11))
 (segment (start 144.2466 95.02) (end 145.276991 95.02) (width 0.25) (layer "F.Cu") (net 11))
 (segment (start 150.9941 100.737109) (end 150.9941 102.8075) (width 0.25) (layer "F.Cu") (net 11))
 (segment (start 144.2466 95.519999) (end 145.140594 95.519999) (width 0.25) (layer "F.Cu") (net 10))
 (segment (start 145.140594 95.519999) (end 148.4541 98.833505) (width 0.25) (layer "F.Cu") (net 10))
 (segment (start 148.4541 98.833505) (end 148.4541 102.8075) (width 0.25) (layer "F.Cu") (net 10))
 (segment (start 145.9141 96.929901) (end 145.9141 102.8075) (width 0.25) (layer "F.Cu") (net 9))
 (segment (start 145.0042 96.020001) (end 145.9141 96.929901) (width 0.25) (layer "F.Cu") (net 9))
 (segment (start 144.2466 96.020001) (end 145.0042 96.020001) (width 0.25) (layer "F.Cu") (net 9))
 (segment (start 143.3741 100.2675) (end 143.3741 102.8075) (width 0.25) (layer "F.Cu") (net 8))
 (segment (start 144.2466 99.395) (end 143.3741 100.2675) (width 0.25) (layer "F.Cu") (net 8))
 (segment (start 144.2466 96.52) (end 144.2466 99.395) (width 0.25) (layer "F.Cu") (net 8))
 (segment (start 143.3741 97.3925) (end 143.3741 98.832079) (width 0.25) (layer "F.Cu") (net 7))
 (segment (start 141.75848 100.447699) (end 140.8341 100.447699) (width 0.25) (layer "F.Cu") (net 7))
 (segment (start 143.3741 98.832079) (end 141.75848 100.447699) (width 0.25) (layer "F.Cu") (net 7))
 (segment (start 140.8341 100.447699) (end 140.8341 102.8075) (width 0.25) (layer "F.Cu") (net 7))
 (segment (start 141.572084 99.997699) (end 138.2941 99.997699) (width 0.25) (layer "F.Cu") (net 6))
 (segment (start 142.874101 98.695682) (end 141.572084 99.997699) (width 0.25) (layer "F.Cu") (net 6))
 (segment (start 142.874101 97.3925) (end 142.874101 98.695682) (width 0.25) (layer "F.Cu") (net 6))
 (segment (start 138.2941 99.997699) (end 138.2941 102.8075) (width 0.25) (layer "F.Cu") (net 6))
 (segment (start 135.7541 99.547699) (end 135.7541 102.8075) (width 0.25) (layer "F.Cu") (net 5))
 (segment (start 142.374099 98.559288) (end 141.385688 99.547699) (width 0.25) (layer "F.Cu") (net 5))
 (segment (start 141.385688 99.547699) (end 135.7541 99.547699) (width 0.25) (layer "F.Cu") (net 5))
 (segment (start 142.374099 97.3925) (end 142.374099 98.559288) (width 0.25) (layer "F.Cu") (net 5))
 (segment (start 141.8741 97.3925) (end 141.8741 98.422891) (width 0.25) (layer "F.Cu") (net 4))
 (segment (start 133.2141 99.097699) (end 133.2141 102.8075) (width 0.25) (layer "F.Cu") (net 4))
 (segment (start 141.8741 98.422891) (end 141.199292 99.097699) (width 0.25) (layer "F.Cu") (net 4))
 (segment (start 141.199292 99.097699) (end 133.2141 99.097699) (width 0.25) (layer "F.Cu") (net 4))
 (segment (start 141.012896 98.647699) (end 130.6741 98.647699) (width 0.25) (layer "F.Cu") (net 3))
 (segment (start 130.6741 98.647699) (end 130.6741 102.8075) (width 0.25) (layer "F.Cu") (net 3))
 (segment (start 141.374101 97.3925) (end 141.374101 98.286494) (width 0.25) (layer "F.Cu") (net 3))
 (segment (start 141.374101 98.286494) (end 141.012896 98.647699) (width 0.25) (layer "F.Cu") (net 3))
 (segment (start 128.1341 98.552898) (end 128.1341 102.8075) (width 0.25) (layer "F.Cu") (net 2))
 (segment (start 140.874099 98.1501) (end 140.8265 98.197699) (width 0.25) (layer "F.Cu") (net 2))
 (segment (start 140.8265 98.197699) (end 128.489299 98.197699) (width 0.25) (layer "F.Cu") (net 2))
 (segment (start 140.874099 97.3925) (end 140.874099 98.1501) (width 0.25) (layer "F.Cu") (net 2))
 (segment (start 128.489299 98.197699) (end 128.1341 98.552898) (width 0.25) (layer "F.Cu") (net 2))
 (segment (start 125.9291 97.3925) (end 125.5941 97.7275) (width 0.25) (layer "F.Cu") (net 1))
 (segment (start 140.3741 97.3925) (end 125.9291 97.3925) (width 0.25) (layer "F.Cu") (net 1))
 (segment (start 125.5941 97.7275) (end 125.5941 102.8075) (width 0.25) (layer "F.Cu") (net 1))
 (segment (start 143.3741 92.6475) (end 158.6141 92.6475) (width 0.25) (layer "F.Cu") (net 15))
 (segment (start 161.1541 90.1075) (end 161.1541 87.5675) (width 0.25) (layer "F.Cu") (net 15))
 (segment (start 158.6141 92.6475) (end 161.1541 90.1075) (width 0.25) (layer "F.Cu") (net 15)))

